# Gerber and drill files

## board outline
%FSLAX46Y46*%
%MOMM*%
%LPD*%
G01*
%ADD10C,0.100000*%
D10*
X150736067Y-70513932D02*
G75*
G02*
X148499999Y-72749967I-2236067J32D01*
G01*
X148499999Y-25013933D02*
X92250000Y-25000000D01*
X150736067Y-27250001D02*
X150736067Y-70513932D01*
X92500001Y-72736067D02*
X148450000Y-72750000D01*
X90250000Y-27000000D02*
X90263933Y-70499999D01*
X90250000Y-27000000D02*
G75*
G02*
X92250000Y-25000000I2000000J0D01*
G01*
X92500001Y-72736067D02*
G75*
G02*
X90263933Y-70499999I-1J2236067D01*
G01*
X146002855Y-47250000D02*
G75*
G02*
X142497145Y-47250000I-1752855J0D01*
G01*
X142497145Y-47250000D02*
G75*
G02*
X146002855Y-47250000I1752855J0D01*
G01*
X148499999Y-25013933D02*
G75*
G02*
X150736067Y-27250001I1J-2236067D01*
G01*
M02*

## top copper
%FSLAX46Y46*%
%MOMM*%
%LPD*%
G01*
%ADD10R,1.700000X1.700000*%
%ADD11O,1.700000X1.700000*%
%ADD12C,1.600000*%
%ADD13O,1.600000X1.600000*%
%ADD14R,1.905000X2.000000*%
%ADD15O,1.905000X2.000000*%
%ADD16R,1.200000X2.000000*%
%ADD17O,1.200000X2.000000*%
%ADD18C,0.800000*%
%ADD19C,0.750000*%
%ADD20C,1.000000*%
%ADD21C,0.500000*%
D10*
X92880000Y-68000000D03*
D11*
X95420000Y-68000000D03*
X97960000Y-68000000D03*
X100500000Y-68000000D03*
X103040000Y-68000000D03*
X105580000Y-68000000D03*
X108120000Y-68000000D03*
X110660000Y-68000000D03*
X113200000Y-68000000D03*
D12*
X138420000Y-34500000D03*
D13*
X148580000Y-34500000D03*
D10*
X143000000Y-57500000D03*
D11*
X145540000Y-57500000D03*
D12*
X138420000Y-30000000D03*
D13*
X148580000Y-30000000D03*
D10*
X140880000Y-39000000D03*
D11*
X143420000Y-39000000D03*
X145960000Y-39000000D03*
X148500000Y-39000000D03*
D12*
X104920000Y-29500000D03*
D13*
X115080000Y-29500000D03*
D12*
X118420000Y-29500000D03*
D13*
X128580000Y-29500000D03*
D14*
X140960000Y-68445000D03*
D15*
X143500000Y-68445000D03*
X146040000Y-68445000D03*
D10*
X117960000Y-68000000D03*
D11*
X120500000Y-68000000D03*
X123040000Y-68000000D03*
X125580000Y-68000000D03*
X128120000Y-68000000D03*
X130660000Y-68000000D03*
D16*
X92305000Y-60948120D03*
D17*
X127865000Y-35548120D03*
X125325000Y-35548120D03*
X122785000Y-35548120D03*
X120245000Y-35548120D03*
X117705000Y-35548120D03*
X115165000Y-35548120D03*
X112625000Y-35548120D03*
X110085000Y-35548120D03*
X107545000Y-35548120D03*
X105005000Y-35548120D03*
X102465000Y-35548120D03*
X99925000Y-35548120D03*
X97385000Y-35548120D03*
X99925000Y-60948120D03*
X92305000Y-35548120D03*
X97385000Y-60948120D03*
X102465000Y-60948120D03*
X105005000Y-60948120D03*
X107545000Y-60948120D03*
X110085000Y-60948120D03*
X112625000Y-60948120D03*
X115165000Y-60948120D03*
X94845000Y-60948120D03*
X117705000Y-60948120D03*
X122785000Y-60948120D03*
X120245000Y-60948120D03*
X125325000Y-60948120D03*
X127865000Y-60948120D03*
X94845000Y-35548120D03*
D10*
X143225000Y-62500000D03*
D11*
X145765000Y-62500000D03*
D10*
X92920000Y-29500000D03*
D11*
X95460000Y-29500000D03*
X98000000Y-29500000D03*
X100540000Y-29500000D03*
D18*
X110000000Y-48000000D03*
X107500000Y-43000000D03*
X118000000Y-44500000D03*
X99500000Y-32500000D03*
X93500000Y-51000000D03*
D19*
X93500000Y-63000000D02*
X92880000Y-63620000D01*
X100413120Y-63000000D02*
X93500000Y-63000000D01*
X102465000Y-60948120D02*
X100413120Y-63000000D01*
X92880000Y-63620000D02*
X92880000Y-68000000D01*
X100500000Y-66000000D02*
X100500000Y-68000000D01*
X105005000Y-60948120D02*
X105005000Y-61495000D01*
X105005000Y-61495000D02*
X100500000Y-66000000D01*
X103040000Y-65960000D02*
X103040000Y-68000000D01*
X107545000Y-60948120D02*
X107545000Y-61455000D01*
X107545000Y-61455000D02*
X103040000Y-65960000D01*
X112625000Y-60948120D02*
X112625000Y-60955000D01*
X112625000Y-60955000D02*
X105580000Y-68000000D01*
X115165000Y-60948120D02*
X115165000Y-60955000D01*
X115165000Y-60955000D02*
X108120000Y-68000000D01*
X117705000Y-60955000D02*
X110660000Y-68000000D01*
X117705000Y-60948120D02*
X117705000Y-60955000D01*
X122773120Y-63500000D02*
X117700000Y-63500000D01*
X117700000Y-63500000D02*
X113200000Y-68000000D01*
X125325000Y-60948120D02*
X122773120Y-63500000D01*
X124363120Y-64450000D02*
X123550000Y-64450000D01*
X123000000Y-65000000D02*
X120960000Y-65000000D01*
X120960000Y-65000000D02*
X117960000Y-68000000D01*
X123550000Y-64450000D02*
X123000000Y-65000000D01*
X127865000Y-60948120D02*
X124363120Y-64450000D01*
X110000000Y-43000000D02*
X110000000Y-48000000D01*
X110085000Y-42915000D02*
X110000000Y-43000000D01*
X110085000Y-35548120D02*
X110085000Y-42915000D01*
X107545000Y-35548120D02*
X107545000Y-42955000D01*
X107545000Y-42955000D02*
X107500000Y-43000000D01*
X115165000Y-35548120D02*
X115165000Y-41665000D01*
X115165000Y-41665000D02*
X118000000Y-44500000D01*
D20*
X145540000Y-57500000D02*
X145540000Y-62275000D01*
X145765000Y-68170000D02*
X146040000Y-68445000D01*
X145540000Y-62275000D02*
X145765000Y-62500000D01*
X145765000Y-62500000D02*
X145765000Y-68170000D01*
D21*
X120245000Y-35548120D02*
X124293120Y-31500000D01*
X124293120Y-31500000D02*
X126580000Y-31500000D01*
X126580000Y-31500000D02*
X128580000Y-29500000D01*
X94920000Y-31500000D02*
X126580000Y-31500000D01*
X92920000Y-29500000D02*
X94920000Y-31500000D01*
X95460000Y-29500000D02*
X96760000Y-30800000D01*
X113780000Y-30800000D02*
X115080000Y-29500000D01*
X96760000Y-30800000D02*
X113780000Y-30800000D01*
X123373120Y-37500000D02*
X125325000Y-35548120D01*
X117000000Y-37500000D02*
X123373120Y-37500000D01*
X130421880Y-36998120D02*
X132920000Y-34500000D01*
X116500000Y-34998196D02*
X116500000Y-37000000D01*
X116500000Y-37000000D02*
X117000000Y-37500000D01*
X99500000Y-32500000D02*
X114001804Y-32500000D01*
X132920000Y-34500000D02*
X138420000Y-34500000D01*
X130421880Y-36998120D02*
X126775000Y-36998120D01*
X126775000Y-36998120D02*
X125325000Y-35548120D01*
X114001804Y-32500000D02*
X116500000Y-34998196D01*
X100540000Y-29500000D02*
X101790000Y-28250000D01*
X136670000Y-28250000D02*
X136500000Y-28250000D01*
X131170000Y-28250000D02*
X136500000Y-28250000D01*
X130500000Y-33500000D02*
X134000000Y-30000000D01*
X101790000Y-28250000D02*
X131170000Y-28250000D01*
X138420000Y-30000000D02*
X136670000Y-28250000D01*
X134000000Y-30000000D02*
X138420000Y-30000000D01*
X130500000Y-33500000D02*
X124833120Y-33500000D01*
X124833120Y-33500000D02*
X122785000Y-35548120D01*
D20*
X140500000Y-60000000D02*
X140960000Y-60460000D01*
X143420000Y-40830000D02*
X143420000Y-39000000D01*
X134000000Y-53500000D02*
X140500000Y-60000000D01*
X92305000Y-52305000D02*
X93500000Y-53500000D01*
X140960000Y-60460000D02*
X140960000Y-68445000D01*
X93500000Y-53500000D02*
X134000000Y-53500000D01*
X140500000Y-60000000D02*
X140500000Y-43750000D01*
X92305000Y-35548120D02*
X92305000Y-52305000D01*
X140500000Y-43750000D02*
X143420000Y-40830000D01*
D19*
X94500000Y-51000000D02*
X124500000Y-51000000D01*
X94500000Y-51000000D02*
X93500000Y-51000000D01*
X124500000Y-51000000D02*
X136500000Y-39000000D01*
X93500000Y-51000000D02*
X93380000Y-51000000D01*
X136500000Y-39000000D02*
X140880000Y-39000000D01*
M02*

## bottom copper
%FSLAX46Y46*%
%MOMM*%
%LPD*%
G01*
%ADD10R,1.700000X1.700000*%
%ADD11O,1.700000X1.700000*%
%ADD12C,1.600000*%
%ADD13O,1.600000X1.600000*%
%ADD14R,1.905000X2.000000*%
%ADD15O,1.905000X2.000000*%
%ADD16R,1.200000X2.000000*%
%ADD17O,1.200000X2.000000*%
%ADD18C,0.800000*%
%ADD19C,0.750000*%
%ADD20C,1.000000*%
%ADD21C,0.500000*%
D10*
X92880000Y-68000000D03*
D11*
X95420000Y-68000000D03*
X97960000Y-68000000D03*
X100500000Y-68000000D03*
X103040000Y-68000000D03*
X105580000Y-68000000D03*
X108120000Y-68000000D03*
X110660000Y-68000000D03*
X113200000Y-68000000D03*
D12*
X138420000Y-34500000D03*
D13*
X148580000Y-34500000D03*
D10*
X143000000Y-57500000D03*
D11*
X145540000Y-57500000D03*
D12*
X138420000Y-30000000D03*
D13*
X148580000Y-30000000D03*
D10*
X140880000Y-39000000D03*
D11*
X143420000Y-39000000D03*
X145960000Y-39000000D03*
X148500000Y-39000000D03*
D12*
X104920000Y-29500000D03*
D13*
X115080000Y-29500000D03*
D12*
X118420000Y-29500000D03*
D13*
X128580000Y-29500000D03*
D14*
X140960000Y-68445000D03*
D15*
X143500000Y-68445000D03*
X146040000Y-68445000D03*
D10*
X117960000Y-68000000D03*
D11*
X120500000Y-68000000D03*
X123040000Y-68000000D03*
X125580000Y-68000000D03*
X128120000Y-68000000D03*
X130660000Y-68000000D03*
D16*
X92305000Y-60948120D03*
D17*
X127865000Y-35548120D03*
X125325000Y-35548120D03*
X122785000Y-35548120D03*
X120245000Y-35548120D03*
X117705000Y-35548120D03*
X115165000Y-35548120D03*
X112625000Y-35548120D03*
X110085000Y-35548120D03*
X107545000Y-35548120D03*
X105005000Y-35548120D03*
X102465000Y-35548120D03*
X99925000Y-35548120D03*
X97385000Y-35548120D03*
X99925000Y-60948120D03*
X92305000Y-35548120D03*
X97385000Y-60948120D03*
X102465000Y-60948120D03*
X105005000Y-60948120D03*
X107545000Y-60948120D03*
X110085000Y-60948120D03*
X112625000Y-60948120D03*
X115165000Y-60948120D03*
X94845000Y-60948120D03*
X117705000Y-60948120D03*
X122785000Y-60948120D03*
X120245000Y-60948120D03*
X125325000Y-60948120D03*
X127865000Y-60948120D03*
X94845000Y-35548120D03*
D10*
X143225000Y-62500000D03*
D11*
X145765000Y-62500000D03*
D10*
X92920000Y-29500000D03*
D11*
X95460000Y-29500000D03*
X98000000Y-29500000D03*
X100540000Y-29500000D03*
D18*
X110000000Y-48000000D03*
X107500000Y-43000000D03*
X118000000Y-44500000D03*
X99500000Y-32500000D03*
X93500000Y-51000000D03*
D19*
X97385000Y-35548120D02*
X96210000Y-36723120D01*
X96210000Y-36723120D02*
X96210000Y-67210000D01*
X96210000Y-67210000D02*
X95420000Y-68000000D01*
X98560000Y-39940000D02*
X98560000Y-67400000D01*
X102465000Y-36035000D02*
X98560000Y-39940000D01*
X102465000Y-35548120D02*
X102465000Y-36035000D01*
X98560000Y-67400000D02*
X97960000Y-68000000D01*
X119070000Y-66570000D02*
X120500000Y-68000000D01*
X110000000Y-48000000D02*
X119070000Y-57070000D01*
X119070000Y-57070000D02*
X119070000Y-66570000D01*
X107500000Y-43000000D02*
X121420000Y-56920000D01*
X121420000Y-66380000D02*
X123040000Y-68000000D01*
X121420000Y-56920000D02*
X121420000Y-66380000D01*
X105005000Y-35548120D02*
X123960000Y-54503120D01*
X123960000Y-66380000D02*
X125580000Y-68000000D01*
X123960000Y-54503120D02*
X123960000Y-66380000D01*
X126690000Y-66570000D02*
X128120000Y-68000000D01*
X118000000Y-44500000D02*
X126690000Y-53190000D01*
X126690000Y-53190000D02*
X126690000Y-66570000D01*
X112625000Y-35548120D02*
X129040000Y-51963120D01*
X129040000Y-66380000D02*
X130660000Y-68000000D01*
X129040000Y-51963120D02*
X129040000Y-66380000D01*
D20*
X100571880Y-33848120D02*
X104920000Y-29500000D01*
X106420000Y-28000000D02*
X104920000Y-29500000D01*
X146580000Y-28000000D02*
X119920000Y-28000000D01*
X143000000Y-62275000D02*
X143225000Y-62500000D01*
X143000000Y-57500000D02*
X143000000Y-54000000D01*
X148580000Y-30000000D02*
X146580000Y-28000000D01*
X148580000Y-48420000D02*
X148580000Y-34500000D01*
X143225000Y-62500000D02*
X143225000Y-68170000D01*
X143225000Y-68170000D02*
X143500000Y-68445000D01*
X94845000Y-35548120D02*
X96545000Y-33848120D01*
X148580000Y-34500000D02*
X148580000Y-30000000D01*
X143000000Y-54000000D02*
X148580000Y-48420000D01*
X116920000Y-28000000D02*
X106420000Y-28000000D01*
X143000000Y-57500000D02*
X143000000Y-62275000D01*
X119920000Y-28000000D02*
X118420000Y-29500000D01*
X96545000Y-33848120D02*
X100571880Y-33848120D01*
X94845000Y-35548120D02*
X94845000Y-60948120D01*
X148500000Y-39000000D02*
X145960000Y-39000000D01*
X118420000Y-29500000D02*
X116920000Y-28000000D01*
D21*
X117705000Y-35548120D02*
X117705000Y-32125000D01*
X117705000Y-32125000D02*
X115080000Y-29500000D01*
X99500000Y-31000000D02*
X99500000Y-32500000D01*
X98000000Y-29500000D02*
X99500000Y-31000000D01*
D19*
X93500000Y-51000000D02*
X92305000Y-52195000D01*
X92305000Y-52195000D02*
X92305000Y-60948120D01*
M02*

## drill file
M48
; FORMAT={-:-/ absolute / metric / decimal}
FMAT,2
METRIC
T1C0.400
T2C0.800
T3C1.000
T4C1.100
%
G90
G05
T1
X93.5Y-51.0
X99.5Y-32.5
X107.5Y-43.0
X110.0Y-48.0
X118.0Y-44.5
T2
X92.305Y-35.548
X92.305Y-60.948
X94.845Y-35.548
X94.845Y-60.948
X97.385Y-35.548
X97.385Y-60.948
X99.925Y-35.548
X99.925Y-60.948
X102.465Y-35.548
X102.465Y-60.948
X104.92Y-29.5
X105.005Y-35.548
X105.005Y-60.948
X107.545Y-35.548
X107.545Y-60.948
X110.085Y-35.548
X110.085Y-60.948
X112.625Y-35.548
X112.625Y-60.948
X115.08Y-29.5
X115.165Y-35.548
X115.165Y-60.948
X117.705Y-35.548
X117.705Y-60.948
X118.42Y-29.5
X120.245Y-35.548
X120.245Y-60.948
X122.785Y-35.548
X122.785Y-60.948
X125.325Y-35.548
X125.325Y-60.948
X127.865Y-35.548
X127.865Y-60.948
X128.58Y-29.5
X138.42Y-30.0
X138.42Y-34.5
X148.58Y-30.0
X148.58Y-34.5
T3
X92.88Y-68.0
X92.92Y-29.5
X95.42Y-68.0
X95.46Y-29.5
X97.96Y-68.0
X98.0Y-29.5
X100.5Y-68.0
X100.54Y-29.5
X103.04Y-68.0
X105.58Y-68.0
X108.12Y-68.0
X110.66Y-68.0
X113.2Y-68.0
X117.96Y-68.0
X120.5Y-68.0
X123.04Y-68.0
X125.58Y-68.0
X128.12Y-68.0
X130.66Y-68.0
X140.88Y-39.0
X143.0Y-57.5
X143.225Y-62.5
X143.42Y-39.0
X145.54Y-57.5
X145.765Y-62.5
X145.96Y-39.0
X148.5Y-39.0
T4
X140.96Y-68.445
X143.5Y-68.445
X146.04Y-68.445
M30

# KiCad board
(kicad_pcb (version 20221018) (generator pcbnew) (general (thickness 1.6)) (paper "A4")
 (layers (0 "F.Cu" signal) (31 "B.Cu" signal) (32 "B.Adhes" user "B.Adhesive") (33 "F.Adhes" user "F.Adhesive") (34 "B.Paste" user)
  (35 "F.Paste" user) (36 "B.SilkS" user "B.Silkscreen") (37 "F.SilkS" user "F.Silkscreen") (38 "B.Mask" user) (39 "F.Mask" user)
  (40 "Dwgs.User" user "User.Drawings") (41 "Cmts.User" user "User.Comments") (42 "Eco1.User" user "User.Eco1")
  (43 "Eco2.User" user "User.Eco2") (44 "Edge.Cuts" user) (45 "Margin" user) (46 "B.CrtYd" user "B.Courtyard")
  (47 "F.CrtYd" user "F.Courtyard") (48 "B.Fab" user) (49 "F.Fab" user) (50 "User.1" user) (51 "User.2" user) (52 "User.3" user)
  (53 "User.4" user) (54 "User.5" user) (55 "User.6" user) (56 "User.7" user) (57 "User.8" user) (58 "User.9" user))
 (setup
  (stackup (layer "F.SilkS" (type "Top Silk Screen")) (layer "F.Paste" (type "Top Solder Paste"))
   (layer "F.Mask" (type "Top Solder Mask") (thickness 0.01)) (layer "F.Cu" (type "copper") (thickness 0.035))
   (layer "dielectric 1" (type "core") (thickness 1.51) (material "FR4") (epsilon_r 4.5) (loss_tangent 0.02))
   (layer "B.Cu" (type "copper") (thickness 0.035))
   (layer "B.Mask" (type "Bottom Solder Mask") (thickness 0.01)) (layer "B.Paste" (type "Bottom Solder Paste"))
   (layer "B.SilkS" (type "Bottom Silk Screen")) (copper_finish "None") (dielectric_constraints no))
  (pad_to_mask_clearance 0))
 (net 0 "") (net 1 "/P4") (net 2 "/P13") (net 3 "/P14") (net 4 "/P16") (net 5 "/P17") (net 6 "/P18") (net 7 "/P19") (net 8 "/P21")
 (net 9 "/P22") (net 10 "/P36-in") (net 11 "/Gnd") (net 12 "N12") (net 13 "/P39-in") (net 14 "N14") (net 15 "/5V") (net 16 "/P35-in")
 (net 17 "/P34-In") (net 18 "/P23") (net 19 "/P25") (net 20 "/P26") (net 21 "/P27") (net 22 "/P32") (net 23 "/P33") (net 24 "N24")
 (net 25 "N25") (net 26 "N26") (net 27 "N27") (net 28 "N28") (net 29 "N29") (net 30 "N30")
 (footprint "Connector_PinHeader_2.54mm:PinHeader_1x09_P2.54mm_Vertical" (layer "F.Cu") (at 92.88 68 90)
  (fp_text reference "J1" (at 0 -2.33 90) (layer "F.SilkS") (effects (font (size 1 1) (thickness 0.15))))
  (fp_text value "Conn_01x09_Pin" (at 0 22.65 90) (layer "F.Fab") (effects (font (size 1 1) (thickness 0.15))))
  (pad "1" thru_hole rect (at 0 0 90) (size 1.7 1.7) (drill 1) (layers "*.Cu" "*.Mask") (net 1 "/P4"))
  (pad "2" thru_hole oval (at 0 2.54 90) (size 1.7 1.7) (drill 1) (layers "*.Cu" "*.Mask") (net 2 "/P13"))
  (pad "3" thru_hole oval (at 0 5.08 90) (size 1.7 1.7) (drill 1) (layers "*.Cu" "*.Mask") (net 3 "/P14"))
  (pad "4" thru_hole oval (at 0 7.62 90) (size 1.7 1.7) (drill 1) (layers "*.Cu" "*.Mask") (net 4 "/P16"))
  (pad "5" thru_hole oval (at 0 10.16 90) (size 1.7 1.7) (drill 1) (layers "*.Cu" "*.Mask") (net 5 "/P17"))
  (pad "6" thru_hole oval (at 0 12.7 90) (size 1.7 1.7) (drill 1) (layers "*.Cu" "*.Mask") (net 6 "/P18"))
  (pad "7" thru_hole oval (at 0 15.24 90) (size 1.7 1.7) (drill 1) (layers "*.Cu" "*.Mask") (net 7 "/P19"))
  (pad "8" thru_hole oval (at 0 17.78 90) (size 1.7 1.7) (drill 1) (layers "*.Cu" "*.Mask") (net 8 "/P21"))
  (pad "9" thru_hole oval (at 0 20.32 90) (size 1.7 1.7) (drill 1) (layers "*.Cu" "*.Mask") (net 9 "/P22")))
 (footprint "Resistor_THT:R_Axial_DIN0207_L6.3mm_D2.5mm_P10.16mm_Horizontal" (layer "F.Cu") (at 138.42 34.5)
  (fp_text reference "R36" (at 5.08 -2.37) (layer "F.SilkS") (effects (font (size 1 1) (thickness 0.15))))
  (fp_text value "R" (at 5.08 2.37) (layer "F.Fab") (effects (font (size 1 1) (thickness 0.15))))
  (pad "1" thru_hole circle (at 0 0) (size 1.6 1.6) (drill 0.8) (layers "*.Cu" "*.Mask") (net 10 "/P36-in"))
  (pad "2" thru_hole oval (at 10.16 0) (size 1.6 1.6) (drill 0.8) (layers "*.Cu" "*.Mask") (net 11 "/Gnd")))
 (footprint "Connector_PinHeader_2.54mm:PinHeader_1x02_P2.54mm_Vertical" (layer "F.Cu") (at 143 57.5 90)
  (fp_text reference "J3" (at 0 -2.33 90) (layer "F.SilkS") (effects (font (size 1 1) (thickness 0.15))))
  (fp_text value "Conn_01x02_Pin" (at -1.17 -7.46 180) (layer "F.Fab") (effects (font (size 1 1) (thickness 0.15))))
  (pad "1" thru_hole rect (at 0 0 90) (size 1.7 1.7) (drill 1) (layers "*.Cu" "*.Mask") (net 11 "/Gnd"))
  (pad "2" thru_hole oval (at 0 2.54 90) (size 1.7 1.7) (drill 1) (layers "*.Cu" "*.Mask") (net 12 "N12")))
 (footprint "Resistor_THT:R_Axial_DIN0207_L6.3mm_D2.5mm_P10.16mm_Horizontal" (layer "F.Cu") (at 138.42 30)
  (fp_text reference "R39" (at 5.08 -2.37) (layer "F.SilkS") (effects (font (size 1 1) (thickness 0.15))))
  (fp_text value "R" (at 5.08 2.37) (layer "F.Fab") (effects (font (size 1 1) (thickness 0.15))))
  (pad "1" thru_hole circle (at 0 0) (size 1.6 1.6) (drill 0.8) (layers "*.Cu" "*.Mask") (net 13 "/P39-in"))
  (pad "2" thru_hole oval (at 10.16 0) (size 1.6 1.6) (drill 0.8) (layers "*.Cu" "*.Mask") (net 11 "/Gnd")))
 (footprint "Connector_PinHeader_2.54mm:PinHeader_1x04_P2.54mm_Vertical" (layer "F.Cu") (at 140.88 39 90)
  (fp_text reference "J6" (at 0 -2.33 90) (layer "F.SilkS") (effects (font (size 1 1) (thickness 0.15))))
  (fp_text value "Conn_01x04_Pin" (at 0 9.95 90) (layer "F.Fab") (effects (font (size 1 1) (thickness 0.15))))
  (pad "1" thru_hole rect (at 0 0 90) (size 1.7 1.7) (drill 1) (layers "*.Cu" "*.Mask") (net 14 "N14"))
  (pad "2" thru_hole oval (at 0 2.54 90) (size 1.7 1.7) (drill 1) (layers "*.Cu" "*.Mask") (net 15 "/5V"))
  (pad "3" thru_hole oval (at 0 5.08 90) (size 1.7 1.7) (drill 1) (layers "*.Cu" "*.Mask") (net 11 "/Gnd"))
  (pad "4" thru_hole oval (at 0 7.62 90) (size 1.7 1.7) (drill 1) (layers "*.Cu" "*.Mask") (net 11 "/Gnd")))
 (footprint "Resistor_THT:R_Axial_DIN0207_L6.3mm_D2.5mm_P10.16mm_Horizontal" (layer "F.Cu") (at 104.92 29.5)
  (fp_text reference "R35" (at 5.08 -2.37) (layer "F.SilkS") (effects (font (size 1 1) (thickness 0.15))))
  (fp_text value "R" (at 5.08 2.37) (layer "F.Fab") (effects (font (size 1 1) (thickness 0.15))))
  (pad "1" thru_hole circle (at 0 0) (size 1.6 1.6) (drill 0.8) (layers "*.Cu" "*.Mask") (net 11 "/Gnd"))
  (pad "2" thru_hole oval (at 10.16 0) (size 1.6 1.6) (drill 0.8) (layers "*.Cu" "*.Mask") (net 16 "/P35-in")))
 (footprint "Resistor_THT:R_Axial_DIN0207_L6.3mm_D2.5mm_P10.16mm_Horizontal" (layer "F.Cu") (at 118.42 29.5)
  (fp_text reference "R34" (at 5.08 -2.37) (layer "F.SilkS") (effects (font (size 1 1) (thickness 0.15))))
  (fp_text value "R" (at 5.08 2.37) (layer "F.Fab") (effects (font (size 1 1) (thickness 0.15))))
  (pad "1" thru_hole circle (at 0 0) (size 1.6 1.6) (drill 0.8) (layers "*.Cu" "*.Mask") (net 11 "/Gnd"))
  (pad "2" thru_hole oval (at 10.16 0) (size 1.6 1.6) (drill 0.8) (layers "*.Cu" "*.Mask") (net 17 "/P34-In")))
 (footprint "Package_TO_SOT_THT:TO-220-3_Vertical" (layer "F.Cu") (at 140.96 68.445)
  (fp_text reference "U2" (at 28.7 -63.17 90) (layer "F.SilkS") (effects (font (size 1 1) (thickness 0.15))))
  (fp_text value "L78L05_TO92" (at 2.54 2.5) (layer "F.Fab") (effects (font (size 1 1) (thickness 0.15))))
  (pad "1" thru_hole rect (at 0 0) (size 1.905 2) (drill 1.1) (layers "*.Cu" "*.Mask") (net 15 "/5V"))
  (pad "2" thru_hole oval (at 2.54 0) (size 1.905 2) (drill 1.1) (layers "*.Cu" "*.Mask") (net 11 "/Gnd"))
  (pad "3" thru_hole oval (at 5.08 0) (size 1.905 2) (drill 1.1) (layers "*.Cu" "*.Mask") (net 12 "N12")))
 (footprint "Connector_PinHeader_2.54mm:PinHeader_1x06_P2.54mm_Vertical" (layer "F.Cu") (at 117.96 68 90)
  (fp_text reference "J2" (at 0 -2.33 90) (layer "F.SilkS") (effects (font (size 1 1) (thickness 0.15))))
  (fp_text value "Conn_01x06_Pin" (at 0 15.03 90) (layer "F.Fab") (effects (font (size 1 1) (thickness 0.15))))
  (pad "1" thru_hole rect (at 0 0 90) (size 1.7 1.7) (drill 1) (layers "*.Cu" "*.Mask") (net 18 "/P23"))
  (pad "2" thru_hole oval (at 0 2.54 90) (size 1.7 1.7) (drill 1) (layers "*.Cu" "*.Mask") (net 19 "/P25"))
  (pad "3" thru_hole oval (at 0 5.08 90) (size 1.7 1.7) (drill 1) (layers "*.Cu" "*.Mask") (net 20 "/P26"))
  (pad "4" thru_hole oval (at 0 7.62 90) (size 1.7 1.7) (drill 1) (layers "*.Cu" "*.Mask") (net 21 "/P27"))
  (pad "5" thru_hole oval (at 0 10.16 90) (size 1.7 1.7) (drill 1) (layers "*.Cu" "*.Mask") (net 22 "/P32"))
  (pad "6" thru_hole oval (at 0 12.7 90) (size 1.7 1.7) (drill 1) (layers "*.Cu" "*.Mask") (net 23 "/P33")))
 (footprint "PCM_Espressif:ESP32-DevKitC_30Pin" (layer "F.Cu") (at 92.305 60.94812 90)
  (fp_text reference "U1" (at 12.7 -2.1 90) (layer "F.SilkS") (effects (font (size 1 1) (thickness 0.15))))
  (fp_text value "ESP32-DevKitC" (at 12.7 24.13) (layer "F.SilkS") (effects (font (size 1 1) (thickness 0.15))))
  (pad "1" thru_hole rect (at 0 0) (size 1.2 2) (drill 0.8) (layers "*.Cu" "*.Mask") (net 14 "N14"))
  (pad "2" thru_hole oval (at 25.4 35.56) (size 1.2 2) (drill 0.8) (layers "*.Cu" "*.Mask") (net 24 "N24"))
  (pad "3" thru_hole oval (at 25.4 33.02) (size 1.2 2) (drill 0.8) (layers "*.Cu" "*.Mask") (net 10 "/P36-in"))
  (pad "4" thru_hole oval (at 25.4 30.48) (size 1.2 2) (drill 0.8) (layers "*.Cu" "*.Mask") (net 13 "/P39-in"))
  (pad "5" thru_hole oval (at 25.4 27.94) (size 1.2 2) (drill 0.8) (layers "*.Cu" "*.Mask") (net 17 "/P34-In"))
  (pad "6" thru_hole oval (at 25.4 25.4) (size 1.2 2) (drill 0.8) (layers "*.Cu" "*.Mask") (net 16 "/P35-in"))
  (pad "7" thru_hole oval (at 25.4 22.86) (size 1.2 2) (drill 0.8) (layers "*.Cu" "*.Mask") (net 22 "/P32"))
  (pad "8" thru_hole oval (at 25.4 20.32) (size 1.2 2) (drill 0.8) (layers "*.Cu" "*.Mask") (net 23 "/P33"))
  (pad "9" thru_hole oval (at 25.4 17.78) (size 1.2 2) (drill 0.8) (layers "*.Cu" "*.Mask") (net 19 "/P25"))
  (pad "10" thru_hole oval (at 25.4 15.24) (size 1.2 2) (drill 0.8) (layers "*.Cu" "*.Mask") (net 20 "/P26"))
  (pad "11" thru_hole oval (at 25.4 12.7) (size 1.2 2) (drill 0.8) (layers "*.Cu" "*.Mask") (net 21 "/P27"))
  (pad "12" thru_hole oval (at 25.4 10.16) (size 1.2 2) (drill 0.8) (layers "*.Cu" "*.Mask") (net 3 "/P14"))
  (pad "13" thru_hole oval (at 25.4 7.62) (size 1.2 2) (drill 0.8) (layers "*.Cu" "*.Mask") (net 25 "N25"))
  (pad "15" thru_hole oval (at 25.4 5.08) (size 1.2 2) (drill 0.8) (layers "*.Cu" "*.Mask") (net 2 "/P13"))
  (pad "16" thru_hole oval (at 0 7.62) (size 1.2 2) (drill 0.8) (layers "*.Cu" "*.Mask") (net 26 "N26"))
  (pad "19" thru_hole oval (at 25.4 0) (size 1.2 2) (drill 0.8) (layers "*.Cu" "*.Mask") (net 15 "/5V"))
  (pad "23" thru_hole oval (at 0 5.08) (size 1.2 2) (drill 0.8) (layers "*.Cu" "*.Mask") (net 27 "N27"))
  (pad "26" thru_hole oval (at 0 10.16) (size 1.2 2) (drill 0.8) (layers "*.Cu" "*.Mask") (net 1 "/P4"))
  (pad "27" thru_hole oval (at 0 12.7) (size 1.2 2) (drill 0.8) (layers "*.Cu" "*.Mask") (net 4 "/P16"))
  (pad "28" thru_hole oval (at 0 15.24) (size 1.2 2) (drill 0.8) (layers "*.Cu" "*.Mask") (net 5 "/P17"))
  (pad "29" thru_hole oval (at 0 17.78) (size 1.2 2) (drill 0.8) (layers "*.Cu" "*.Mask") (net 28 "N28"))
  (pad "30" thru_hole oval (at 0 20.32) (size 1.2 2) (drill 0.8) (layers "*.Cu" "*.Mask") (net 6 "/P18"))
  (pad "31" thru_hole oval (at 0 22.86) (size 1.2 2) (drill 0.8) (layers "*.Cu" "*.Mask") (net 7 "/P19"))
  (pad "32" thru_hole oval (at 0 2.54) (size 1.2 2) (drill 0.8) (layers "*.Cu" "*.Mask") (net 11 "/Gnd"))
  (pad "33" thru_hole oval (at 0 25.4) (size 1.2 2) (drill 0.8) (layers "*.Cu" "*.Mask") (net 8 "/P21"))
  (pad "34" thru_hole oval (at 0 30.48) (size 1.2 2) (drill 0.8) (layers "*.Cu" "*.Mask") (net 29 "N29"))
  (pad "35" thru_hole oval (at 0 27.94) (size 1.2 2) (drill 0.8) (layers "*.Cu" "*.Mask") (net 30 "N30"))
  (pad "36" thru_hole oval (at 0 33.02) (size 1.2 2) (drill 0.8) (layers "*.Cu" "*.Mask") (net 9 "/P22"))
  (pad "37" thru_hole oval (at 0 35.56) (size 1.2 2) (drill 0.8) (layers "*.Cu" "*.Mask") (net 18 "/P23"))
  (pad "38" thru_hole oval (at 25.4 2.54) (size 1.2 2) (drill 0.8) (layers "*.Cu" "*.Mask") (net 11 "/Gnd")))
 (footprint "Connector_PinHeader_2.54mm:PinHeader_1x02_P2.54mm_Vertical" (layer "F.Cu") (at 143.225 62.5 90)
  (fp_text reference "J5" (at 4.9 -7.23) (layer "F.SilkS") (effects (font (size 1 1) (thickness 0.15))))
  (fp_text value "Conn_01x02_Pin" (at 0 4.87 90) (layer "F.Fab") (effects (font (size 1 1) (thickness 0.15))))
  (pad "1" thru_hole rect (at 0 0 90) (size 1.7 1.7) (drill 1) (layers "*.Cu" "*.Mask") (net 11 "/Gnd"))
  (pad "2" thru_hole oval (at 0 2.54 90) (size 1.7 1.7) (drill 1) (layers "*.Cu" "*.Mask") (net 12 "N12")))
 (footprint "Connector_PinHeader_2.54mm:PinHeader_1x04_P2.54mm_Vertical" (layer "F.Cu") (at 92.92 29.5 90)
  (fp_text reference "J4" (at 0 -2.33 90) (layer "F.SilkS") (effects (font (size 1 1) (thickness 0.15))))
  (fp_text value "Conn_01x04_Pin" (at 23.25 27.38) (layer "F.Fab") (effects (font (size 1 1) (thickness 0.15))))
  (pad "1" thru_hole rect (at 0 0 90) (size 1.7 1.7) (drill 1) (layers "*.Cu" "*.Mask") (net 17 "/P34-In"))
  (pad "2" thru_hole oval (at 0 2.54 90) (size 1.7 1.7) (drill 1) (layers "*.Cu" "*.Mask") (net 16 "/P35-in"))
  (pad "3" thru_hole oval (at 0 5.08 90) (size 1.7 1.7) (drill 1) (layers "*.Cu" "*.Mask") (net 10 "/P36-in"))
  (pad "4" thru_hole oval (at 0 7.62 90) (size 1.7 1.7) (drill 1) (layers "*.Cu" "*.Mask") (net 13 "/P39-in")))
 (gr_arc (start 150.736067 70.513932) (mid 150.081138 72.095071) (end 148.499999 72.75) (stroke (width 0.1) (type default))
  (layer "Edge.Cuts"))
 (gr_line (start 148.499999 25.013933) (end 92.25 25) (stroke (width 0.1) (type default)) (layer "Edge.Cuts"))
 (gr_line (start 150.736067 27.250001) (end 150.736067 70.513932) (stroke (width 0.1) (type default)) (layer "Edge.Cuts"))
 (gr_line (start 92.500001 72.736067) (end 148.45 72.75) (stroke (width 0.1) (type default)) (layer "Edge.Cuts"))
 (gr_line (start 90.25 27) (end 90.263933 70.499999) (stroke (width 0.1) (type default)) (layer "Edge.Cuts"))
 (gr_arc (start 90.25 27) (mid 90.835786 25.585786) (end 92.25 25) (stroke (width 0.1) (type default)) (layer "Edge.Cuts"))
 (gr_arc (start 92.500001 72.736067) (mid 90.918862 72.081138) (end 90.263933 70.499999) (stroke (width 0.1) (type default))
  (layer "Edge.Cuts"))
 (gr_circle (center 144.25 47.25) (end 146 47.15) (stroke (width 0.1) (type default)) (fill none) (layer "Edge.Cuts"))
 (gr_arc (start 148.499999 25.013933) (mid 150.081138 25.668862) (end 150.736067 27.250001) (stroke (width 0.1) (type default))
  (layer "Edge.Cuts"))
 (segment (start 93.5 63) (end 92.88 63.62) (width 0.75) (layer "F.Cu") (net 1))
 (segment (start 100.41312 63) (end 93.5 63) (width 0.75) (layer "F.Cu") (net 1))
 (segment (start 102.465 60.94812) (end 100.41312 63) (width 0.75) (layer "F.Cu") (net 1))
 (segment (start 92.88 63.62) (end 92.88 68) (width 0.75) (layer "F.Cu") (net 1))
 (segment (start 97.385 35.54812) (end 96.21 36.72312) (width 0.75) (layer "B.Cu") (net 2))
 (segment (start 96.21 36.72312) (end 96.21 67.21) (width 0.75) (layer "B.Cu") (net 2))
 (segment (start 96.21 67.21) (end 95.42 68) (width 0.75) (layer "B.Cu") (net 2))
 (segment (start 98.56 39.94) (end 98.56 67.4) (width 0.75) (layer "B.Cu") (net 3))
 (segment (start 102.465 36.035) (end 98.56 39.94) (width 0.75) (layer "B.Cu") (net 3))
 (segment (start 102.465 35.54812) (end 102.465 36.035) (width 0.75) (layer "B.Cu") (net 3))
 (segment (start 98.56 67.4) (end 97.96 68) (width 0.75) (layer "B.Cu") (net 3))
 (segment (start 100.5 66) (end 100.5 68) (width 0.75) (layer "F.Cu") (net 4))
 (segment (start 105.005 60.94812) (end 105.005 61.495) (width 0.75) (layer "F.Cu") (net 4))
 (segment (start 105.005 61.495) (end 100.5 66) (width 0.75) (layer "F.Cu") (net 4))
 (segment (start 103.04 65.96) (end 103.04 68) (width 0.75) (layer "F.Cu") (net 5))
 (segment (start 107.545 60.94812) (end 107.545 61.455) (width 0.75) (layer "F.Cu") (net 5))
 (segment (start 107.545 61.455) (end 103.04 65.96) (width 0.75) (layer "F.Cu") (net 5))
 (segment (start 112.625 60.94812) (end 112.625 60.955) (width 0.75) (layer "F.Cu") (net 6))
 (segment (start 112.625 60.955) (end 105.58 68) (width 0.75) (layer "F.Cu") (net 6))
 (segment (start 115.165 60.94812) (end 115.165 60.955) (width 0.75) (layer "F.Cu") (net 7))
 (segment (start 115.165 60.955) (end 108.12 68) (width 0.75) (layer "F.Cu") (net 7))
 (segment (start 117.705 60.955) (end 110.66 68) (width 0.75) (layer "F.Cu") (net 8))
 (segment (start 117.705 60.94812) (end 117.705 60.955) (width 0.75) (layer "F.Cu") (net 8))
 (segment (start 122.77312 63.5) (end 117.7 63.5) (width 0.75) (layer "F.Cu") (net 9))
 (segment (start 117.7 63.5) (end 113.2 68) (width 0.75) (layer "F.Cu") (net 9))
 (segment (start 125.325 60.94812) (end 122.77312 63.5) (width 0.75) (layer "F.Cu") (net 9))
 (segment (start 124.36312 64.45) (end 123.55 64.45) (width 0.75) (layer "F.Cu") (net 18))
 (segment (start 123 65) (end 120.96 65) (width 0.75) (layer "F.Cu") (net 18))
 (segment (start 120.96 65) (end 117.96 68) (width 0.75) (layer "F.Cu") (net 18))
 (segment (start 123.55 64.45) (end 123 65) (width 0.75) (layer "F.Cu") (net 18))
 (segment (start 127.865 60.94812) (end 124.36312 64.45) (width 0.75) (layer "F.Cu") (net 18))
 (segment (start 110 43) (end 110 48) (width 0.75) (layer "F.Cu") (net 19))
 (segment (start 110.085 42.915) (end 110 43) (width 0.75) (layer "F.Cu") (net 19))
 (segment (start 110.085 35.54812) (end 110.085 42.915) (width 0.75) (layer "F.Cu") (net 19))
 (via (at 110 48) (size 0.8) (drill 0.4) (layers "F.Cu" "B.Cu") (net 19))
 (segment (start 119.07 66.57) (end 120.5 68) (width 0.75) (layer "B.Cu") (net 19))
 (segment (start 110 48) (end 119.07 57.07) (width 0.75) (layer "B.Cu") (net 19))
 (segment (start 119.07 57.07) (end 119.07 66.57) (width 0.75) (layer "B.Cu") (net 19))
 (segment (start 107.545 35.54812) (end 107.545 42.955) (width 0.75) (layer "F.Cu") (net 20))
 (segment (start 107.545 42.955) (end 107.5 43) (width 0.75) (layer "F.Cu") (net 20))
 (via (at 107.5 43) (size 0.8) (drill 0.4) (layers "F.Cu" "B.Cu") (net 20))
 (segment (start 107.5 43) (end 121.42 56.92) (width 0.75) (layer "B.Cu") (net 20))
 (segment (start 121.42 66.38) (end 123.04 68) (width 0.75) (layer "B.Cu") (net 20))
 (segment (start 121.42 56.92) (end 121.42 66.38) (width 0.75) (layer "B.Cu") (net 20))
 (segment (start 105.005 35.54812) (end 123.96 54.50312) (width 0.75) (layer "B.Cu") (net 21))
 (segment (start 123.96 66.38) (end 125.58 68) (width 0.75) (layer "B.Cu") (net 21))
 (segment (start 123.96 54.50312) (end 123.96 66.38) (width 0.75) (layer "B.Cu") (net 21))
 (segment (start 115.165 35.54812) (end 115.165 41.665) (width 0.75) (layer "F.Cu") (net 22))
 (segment (start 115.165 41.665) (end 118 44.5) (width 0.75) (layer "F.Cu") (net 22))
 (via (at 118 44.5) (size 0.8) (drill 0.4) (layers "F.Cu" "B.Cu") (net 22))
 (segment (start 126.69 66.57) (end 128.12 68) (width 0.75) (layer "B.Cu") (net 22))
 (segment (start 118 44.5) (end 126.69 53.19) (width 0.75) (layer "B.Cu") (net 22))
 (segment (start 126.69 53.19) (end 126.69 66.57) (width 0.75) (layer "B.Cu") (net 22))
 (segment (start 112.625 35.54812) (end 129.04 51.96312) (width 0.75) (layer "B.Cu") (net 23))
 (segment (start 129.04 66.38) (end 130.66 68) (width 0.75) (layer "B.Cu") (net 23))
 (segment (start 129.04 51.96312) (end 129.04 66.38) (width 0.75) (layer "B.Cu") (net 23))
 (segment (start 100.57188 33.84812) (end 104.92 29.5) (width 1) (layer "B.Cu") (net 11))
 (segment (start 106.42 28) (end 104.92 29.5) (width 1) (layer "B.Cu") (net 11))
 (segment (start 146.58 28) (end 119.92 28) (width 1) (layer "B.Cu") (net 11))
 (segment (start 143 62.275) (end 143.225 62.5) (width 1) (layer "B.Cu") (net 11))
 (segment (start 143 57.5) (end 143 54) (width 1) (layer "B.Cu") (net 11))
 (segment (start 148.58 30) (end 146.58 28) (width 1) (layer "B.Cu") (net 11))
 (segment (start 148.58 48.42) (end 148.58 34.5) (width 1) (layer "B.Cu") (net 11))
 (segment (start 143.225 62.5) (end 143.225 68.17) (width 1) (layer "B.Cu") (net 11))
 (segment (start 143.225 68.17) (end 143.5 68.445) (width 1) (layer "B.Cu") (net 11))
 (segment (start 94.845 35.54812) (end 96.545 33.84812) (width 1) (layer "B.Cu") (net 11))
 (segment (start 148.58 34.5) (end 148.58 30) (width 1) (layer "B.Cu") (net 11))
 (segment (start 143 54) (end 148.58 48.42) (width 1) (layer "B.Cu") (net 11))
 (segment (start 116.92 28) (end 106.42 28) (width 1) (layer "B.Cu") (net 11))
 (segment (start 143 57.5) (end 143 62.275) (width 1) (layer "B.Cu") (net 11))
 (segment (start 119.92 28) (end 118.42 29.5) (width 1) (layer "B.Cu") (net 11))
 (segment (start 96.545 33.84812) (end 100.57188 33.84812) (width 1) (layer "B.Cu") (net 11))
 (segment (start 94.845 35.54812) (end 94.845 60.94812) (width 1) (layer "B.Cu") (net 11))
 (segment (start 148.5 39) (end 145.96 39) (width 1) (layer "B.Cu") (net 11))
 (segment (start 118.42 29.5) (end 116.92 28) (width 1) (layer "B.Cu") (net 11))
 (segment (start 145.54 57.5) (end 145.54 62.275) (width 1) (layer "F.Cu") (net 12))
 (segment (start 145.765 68.17) (end 146.04 68.445) (width 1) (layer "F.Cu") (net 12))
 (segment (start 145.54 62.275) (end 145.765 62.5) (width 1) (layer "F.Cu") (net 12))
 (segment (start 145.765 62.5) (end 145.765 68.17) (width 1) (layer "F.Cu") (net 12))
 (segment (start 120.245 35.54812) (end 124.29312 31.5) (width 0.5) (layer "F.Cu") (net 17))
 (segment (start 124.29312 31.5) (end 126.58 31.5) (width 0.5) (layer "F.Cu") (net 17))
 (segment (start 126.58 31.5) (end 128.58 29.5) (width 0.5) (layer "F.Cu") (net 17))
 (segment (start 94.92 31.5) (end 126.58 31.5) (width 0.5) (layer "F.Cu") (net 17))
 (segment (start 92.92 29.5) (end 94.92 31.5) (width 0.5) (layer "F.Cu") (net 17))
 (segment (start 95.46 29.5) (end 96.76 30.8) (width 0.5) (layer "F.Cu") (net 16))
 (segment (start 113.78 30.8) (end 115.08 29.5) (width 0.5) (layer "F.Cu") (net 16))
 (segment (start 96.76 30.8) (end 113.78 30.8) (width 0.5) (layer "F.Cu") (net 16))
 (segment (start 117.705 35.54812) (end 117.705 32.125) (width 0.5) (layer "B.Cu") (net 16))
 (segment (start 117.705 32.125) (end 115.08 29.5) (width 0.5) (layer "B.Cu") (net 16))
 (segment (start 123.37312 37.5) (end 125.325 35.54812) (width 0.5) (layer "F.Cu") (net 10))
 (segment (start 117 37.5) (end 123.37312 37.5) (width 0.5) (layer "F.Cu") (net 10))
 (segment (start 130.42188 36.99812) (end 132.92 34.5) (width 0.5) (layer "F.Cu") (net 10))
 (segment (start 116.5 34.998196) (end 116.5 37) (width 0.5) (layer "F.Cu") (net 10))
 (segment (start 116.5 37) (end 117 37.5) (width 0.5) (layer "F.Cu") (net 10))
 (segment (start 99.5 32.5) (end 114.001804 32.5) (width 0.5) (layer "F.Cu") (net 10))
 (segment (start 132.92 34.5) (end 138.42 34.5) (width 0.5) (layer "F.Cu") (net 10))
 (segment (start 130.42188 36.99812) (end 126.775 36.99812) (width 0.5) (layer "F.Cu") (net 10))
 (segment (start 126.775 36.99812) (end 125.325 35.54812) (width 0.5) (layer "F.Cu") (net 10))
 (segment (start 114.001804 32.5) (end 116.5 34.998196) (width 0.5) (layer "F.Cu") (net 10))
 (via (at 99.5 32.5) (size 0.8) (drill 0.4) (layers "F.Cu" "B.Cu") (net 10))
 (segment (start 99.5 31) (end 99.5 32.5) (width 0.5) (layer "B.Cu") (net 10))
 (segment (start 98 29.5) (end 99.5 31) (width 0.5) (layer "B.Cu") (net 10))
 (segment (start 100.54 29.5) (end 101.79 28.25) (width 0.5) (layer "F.Cu") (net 13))
 (segment (start 136.67 28.25) (end 136.5 28.25) (width 0.5) (layer "F.Cu") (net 13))
 (segment (start 131.17 28.25) (end 136.5 28.25) (width 0.5) (layer "F.Cu") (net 13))
 (segment (start 130.5 33.5) (end 134 30) (width 0.5) (layer "F.Cu") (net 13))
 (segment (start 101.79 28.25) (end 131.17 28.25) (width 0.5) (layer "F.Cu") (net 13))
 (segment (start 138.42 30) (end 136.67 28.25) (width 0.5) (layer "F.Cu") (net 13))
 (segment (start 134 30) (end 138.42 30) (width 0.5) (layer "F.Cu") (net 13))
 (segment (start 130.5 33.5) (end 124.83312 33.5) (width 0.5) (layer "F.Cu") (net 13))
 (segment (start 124.83312 33.5) (end 122.785 35.54812) (width 0.5) (layer "F.Cu") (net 13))
 (segment (start 140.5 60) (end 140.96 60.46) (width 1) (layer "F.Cu") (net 15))
 (segment (start 143.42 40.83) (end 143.42 39) (width 1) (layer "F.Cu") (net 15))
 (segment (start 134 53.5) (end 140.5 60) (width 1) (layer "F.Cu") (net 15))
 (segment (start 92.305 52.305) (end 93.5 53.5) (width 1) (layer "F.Cu") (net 15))
 (segment (start 140.96 60.46) (end 140.96 68.445) (width 1) (layer "F.Cu") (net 15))
 (segment (start 93.5 53.5) (end 134 53.5) (width 1) (layer "F.Cu") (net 15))
 (segment (start 140.5 60) (end 140.5 43.75) (width 1) (layer "F.Cu") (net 15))
 (segment (start 92.305 35.54812) (end 92.305 52.305) (width 1) (layer "F.Cu") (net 15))
 (segment (start 140.5 43.75) (end 143.42 40.83) (width 1) (layer "F.Cu") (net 15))
 (segment (start 94.5 51) (end 124.5 51) (width 0.75) (layer "F.Cu") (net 14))
 (segment (start 94.5 51) (end 93.5 51) (width 0.75) (layer "F.Cu") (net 14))
 (segment (start 124.5 51) (end 136.5 39) (width 0.75) (layer "F.Cu") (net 14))
 (segment (start 93.5 51) (end 93.38 51) (width 0.75) (layer "F.Cu") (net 14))
 (segment (start 136.5 39) (end 140.88 39) (width 0.75) (layer "F.Cu") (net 14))
 (via (at 93.5 51) (size 0.8) (drill 0.4) (layers "F.Cu" "B.Cu") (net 14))
 (segment (start 93.5 51) (end 92.305 52.195) (width 0.75) (layer "B.Cu") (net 14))
 (segment (start 92.305 52.195) (end 92.305 60.94812) (width 0.75) (layer "B.Cu") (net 14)))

